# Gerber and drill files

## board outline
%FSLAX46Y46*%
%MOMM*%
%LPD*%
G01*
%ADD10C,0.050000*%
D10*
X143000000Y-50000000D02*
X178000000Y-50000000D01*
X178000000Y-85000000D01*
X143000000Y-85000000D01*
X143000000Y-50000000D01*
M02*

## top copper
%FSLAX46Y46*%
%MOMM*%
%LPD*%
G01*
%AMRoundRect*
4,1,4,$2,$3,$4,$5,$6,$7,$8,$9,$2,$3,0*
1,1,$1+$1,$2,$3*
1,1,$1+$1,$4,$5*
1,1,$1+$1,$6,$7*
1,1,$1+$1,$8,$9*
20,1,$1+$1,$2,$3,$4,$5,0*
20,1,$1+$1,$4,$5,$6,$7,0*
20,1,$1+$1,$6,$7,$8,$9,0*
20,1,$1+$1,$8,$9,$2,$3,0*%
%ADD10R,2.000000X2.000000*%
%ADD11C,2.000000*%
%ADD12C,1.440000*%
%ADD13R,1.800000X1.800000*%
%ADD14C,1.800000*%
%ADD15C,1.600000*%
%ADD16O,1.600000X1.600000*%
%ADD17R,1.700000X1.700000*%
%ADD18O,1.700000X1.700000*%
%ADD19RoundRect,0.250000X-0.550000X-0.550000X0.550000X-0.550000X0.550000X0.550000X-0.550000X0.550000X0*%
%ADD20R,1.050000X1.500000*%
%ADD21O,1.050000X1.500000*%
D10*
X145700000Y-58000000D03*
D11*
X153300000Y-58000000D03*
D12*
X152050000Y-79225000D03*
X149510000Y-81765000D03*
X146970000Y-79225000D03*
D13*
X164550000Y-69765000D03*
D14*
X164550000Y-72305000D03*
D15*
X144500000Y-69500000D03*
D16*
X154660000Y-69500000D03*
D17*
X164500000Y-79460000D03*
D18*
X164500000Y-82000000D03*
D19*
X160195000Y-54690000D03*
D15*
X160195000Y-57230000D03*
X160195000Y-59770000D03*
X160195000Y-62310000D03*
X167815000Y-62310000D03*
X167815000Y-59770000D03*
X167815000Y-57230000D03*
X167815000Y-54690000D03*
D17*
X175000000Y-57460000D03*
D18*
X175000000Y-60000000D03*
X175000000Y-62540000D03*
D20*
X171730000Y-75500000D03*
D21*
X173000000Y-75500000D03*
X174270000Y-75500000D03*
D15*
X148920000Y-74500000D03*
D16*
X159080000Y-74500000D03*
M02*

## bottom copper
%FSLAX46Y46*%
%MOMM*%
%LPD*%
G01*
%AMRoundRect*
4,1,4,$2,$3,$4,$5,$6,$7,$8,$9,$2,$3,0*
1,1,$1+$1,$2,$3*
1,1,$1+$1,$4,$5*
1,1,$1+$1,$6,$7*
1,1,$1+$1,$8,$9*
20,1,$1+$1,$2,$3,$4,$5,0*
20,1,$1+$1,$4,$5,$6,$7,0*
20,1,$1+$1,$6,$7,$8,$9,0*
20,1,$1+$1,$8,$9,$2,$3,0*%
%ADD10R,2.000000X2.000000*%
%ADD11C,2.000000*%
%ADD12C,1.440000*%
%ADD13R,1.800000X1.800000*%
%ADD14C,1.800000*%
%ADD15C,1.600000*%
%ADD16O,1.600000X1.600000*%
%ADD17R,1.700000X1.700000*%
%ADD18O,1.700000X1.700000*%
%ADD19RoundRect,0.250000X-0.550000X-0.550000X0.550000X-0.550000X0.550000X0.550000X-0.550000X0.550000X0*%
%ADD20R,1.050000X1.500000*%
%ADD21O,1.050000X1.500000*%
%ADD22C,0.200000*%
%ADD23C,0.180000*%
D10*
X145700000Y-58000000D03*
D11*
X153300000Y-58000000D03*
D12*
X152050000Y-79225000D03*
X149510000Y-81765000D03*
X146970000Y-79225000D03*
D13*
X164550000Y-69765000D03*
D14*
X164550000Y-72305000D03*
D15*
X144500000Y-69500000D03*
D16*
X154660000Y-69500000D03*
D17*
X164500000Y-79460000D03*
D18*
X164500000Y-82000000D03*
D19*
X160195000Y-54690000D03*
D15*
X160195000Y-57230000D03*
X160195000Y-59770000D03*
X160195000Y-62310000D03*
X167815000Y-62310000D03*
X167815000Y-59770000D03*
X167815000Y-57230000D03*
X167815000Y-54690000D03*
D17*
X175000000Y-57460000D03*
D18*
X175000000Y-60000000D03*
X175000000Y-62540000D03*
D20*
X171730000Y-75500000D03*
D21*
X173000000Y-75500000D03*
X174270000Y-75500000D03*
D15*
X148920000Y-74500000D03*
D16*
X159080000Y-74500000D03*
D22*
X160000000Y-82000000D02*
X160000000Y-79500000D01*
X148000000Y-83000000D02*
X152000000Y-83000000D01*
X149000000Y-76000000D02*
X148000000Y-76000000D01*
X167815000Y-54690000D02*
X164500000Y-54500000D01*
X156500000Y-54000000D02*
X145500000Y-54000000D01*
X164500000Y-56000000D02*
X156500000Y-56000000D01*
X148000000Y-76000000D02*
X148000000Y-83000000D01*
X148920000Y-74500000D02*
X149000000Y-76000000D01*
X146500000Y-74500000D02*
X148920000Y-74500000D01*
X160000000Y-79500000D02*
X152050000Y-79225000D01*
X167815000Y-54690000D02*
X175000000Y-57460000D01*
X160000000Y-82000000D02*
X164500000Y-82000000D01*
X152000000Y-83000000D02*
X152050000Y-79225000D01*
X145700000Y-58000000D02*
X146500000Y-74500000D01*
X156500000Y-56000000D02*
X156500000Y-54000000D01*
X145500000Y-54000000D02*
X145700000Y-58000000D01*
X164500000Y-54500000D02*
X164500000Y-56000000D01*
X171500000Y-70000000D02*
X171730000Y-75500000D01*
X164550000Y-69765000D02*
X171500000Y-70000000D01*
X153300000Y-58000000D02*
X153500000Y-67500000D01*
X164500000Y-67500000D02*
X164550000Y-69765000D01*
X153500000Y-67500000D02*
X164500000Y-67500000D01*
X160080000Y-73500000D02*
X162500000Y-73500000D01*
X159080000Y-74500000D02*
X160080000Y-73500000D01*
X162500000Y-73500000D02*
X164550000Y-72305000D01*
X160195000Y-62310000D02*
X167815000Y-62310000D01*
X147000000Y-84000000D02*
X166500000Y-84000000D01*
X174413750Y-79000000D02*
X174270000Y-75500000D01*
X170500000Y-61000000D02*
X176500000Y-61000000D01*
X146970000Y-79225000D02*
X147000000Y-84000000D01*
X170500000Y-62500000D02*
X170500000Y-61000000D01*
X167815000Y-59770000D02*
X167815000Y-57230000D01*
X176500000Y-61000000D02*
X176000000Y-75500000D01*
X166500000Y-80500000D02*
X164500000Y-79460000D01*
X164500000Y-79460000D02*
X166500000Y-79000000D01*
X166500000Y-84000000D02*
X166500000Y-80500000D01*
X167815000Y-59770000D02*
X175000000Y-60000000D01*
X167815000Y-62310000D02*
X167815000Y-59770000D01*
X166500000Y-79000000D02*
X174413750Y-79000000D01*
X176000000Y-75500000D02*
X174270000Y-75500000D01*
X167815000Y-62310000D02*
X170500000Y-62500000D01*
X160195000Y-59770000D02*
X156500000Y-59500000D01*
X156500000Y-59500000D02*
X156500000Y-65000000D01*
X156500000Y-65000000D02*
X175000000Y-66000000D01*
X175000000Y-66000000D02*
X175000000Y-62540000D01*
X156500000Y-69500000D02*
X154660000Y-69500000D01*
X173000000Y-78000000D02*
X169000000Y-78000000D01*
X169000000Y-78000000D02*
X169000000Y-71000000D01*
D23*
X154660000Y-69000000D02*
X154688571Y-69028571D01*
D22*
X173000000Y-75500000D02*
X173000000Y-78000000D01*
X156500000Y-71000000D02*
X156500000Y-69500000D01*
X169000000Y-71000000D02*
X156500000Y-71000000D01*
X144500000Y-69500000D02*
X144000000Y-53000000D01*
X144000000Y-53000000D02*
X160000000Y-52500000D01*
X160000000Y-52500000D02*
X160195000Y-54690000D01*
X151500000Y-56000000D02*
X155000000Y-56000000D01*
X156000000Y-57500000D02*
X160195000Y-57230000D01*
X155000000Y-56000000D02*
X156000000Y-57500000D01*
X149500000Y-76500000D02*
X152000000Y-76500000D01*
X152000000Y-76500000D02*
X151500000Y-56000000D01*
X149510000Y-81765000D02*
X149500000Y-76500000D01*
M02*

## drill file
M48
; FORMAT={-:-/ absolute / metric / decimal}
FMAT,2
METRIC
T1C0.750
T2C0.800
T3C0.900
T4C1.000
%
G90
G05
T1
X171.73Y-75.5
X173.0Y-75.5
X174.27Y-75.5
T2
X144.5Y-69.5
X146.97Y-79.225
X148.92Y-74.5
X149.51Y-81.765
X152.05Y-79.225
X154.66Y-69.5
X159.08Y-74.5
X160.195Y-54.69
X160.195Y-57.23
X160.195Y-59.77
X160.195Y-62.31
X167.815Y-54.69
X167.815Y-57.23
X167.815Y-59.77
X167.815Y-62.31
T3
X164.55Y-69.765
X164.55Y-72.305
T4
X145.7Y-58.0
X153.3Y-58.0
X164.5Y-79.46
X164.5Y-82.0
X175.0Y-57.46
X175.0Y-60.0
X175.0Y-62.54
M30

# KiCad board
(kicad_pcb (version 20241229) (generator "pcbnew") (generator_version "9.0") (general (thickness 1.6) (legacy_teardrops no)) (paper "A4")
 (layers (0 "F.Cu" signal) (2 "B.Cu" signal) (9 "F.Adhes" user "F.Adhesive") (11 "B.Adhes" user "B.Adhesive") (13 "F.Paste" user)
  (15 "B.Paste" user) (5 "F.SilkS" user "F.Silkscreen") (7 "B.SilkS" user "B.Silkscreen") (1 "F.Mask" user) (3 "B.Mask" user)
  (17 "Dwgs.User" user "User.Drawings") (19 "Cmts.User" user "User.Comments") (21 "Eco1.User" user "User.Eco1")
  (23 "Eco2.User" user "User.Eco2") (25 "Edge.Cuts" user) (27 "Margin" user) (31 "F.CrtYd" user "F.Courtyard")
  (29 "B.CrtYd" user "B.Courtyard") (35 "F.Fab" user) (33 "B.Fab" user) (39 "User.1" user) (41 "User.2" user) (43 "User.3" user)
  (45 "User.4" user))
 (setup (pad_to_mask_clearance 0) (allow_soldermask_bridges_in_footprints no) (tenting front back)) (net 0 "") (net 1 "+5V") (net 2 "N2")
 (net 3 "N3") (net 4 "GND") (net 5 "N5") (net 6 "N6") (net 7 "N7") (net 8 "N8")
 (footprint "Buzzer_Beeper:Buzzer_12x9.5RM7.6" (layer "F.Cu") (at 145.7 58)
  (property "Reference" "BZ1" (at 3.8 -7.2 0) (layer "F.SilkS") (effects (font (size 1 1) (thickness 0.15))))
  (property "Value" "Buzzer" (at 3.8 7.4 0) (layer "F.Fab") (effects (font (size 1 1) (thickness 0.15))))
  (pad "1" thru_hole rect (at 0 0) (size 2 2) (drill 1) (layers "*.Cu" "*.Mask") (remove_unused_layers no) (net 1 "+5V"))
  (pad "2" thru_hole circle (at 7.6 0) (size 2 2) (drill 1) (layers "*.Cu" "*.Mask") (remove_unused_layers no) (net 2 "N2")))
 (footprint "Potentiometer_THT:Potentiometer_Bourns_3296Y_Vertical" (layer "F.Cu") (at 152.05 79.225)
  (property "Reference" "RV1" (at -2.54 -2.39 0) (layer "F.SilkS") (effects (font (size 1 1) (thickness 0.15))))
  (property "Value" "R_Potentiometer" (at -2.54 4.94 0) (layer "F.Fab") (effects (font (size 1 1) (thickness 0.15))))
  (pad "1" thru_hole circle (at 0 0) (size 1.44 1.44) (drill 0.8) (layers "*.Cu" "*.Mask") (remove_unused_layers no) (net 1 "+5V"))
  (pad "2" thru_hole circle (at -2.54 2.54) (size 1.44 1.44) (drill 0.8) (layers "*.Cu" "*.Mask") (remove_unused_layers no) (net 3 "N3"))
  (pad "3" thru_hole circle (at -5.08 0) (size 1.44 1.44) (drill 0.8) (layers "*.Cu" "*.Mask") (remove_unused_layers no) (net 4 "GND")))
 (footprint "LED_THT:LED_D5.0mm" (layer "F.Cu") (at 164.55 69.765 -90)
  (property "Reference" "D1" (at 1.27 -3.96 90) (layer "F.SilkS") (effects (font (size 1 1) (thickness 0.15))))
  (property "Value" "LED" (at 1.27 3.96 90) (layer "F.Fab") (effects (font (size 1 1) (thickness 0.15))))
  (pad "1" thru_hole rect (at 0 0 270) (size 1.8 1.8) (drill 0.9) (layers "*.Cu" "*.Mask") (remove_unused_layers no) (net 2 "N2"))
  (pad "2" thru_hole circle (at 2.54 0 270) (size 1.8 1.8) (drill 0.9) (layers "*.Cu" "*.Mask") (remove_unused_layers no) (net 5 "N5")))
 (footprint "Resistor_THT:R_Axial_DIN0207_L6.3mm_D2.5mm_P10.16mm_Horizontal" (layer "F.Cu") (at 144.5 69.5)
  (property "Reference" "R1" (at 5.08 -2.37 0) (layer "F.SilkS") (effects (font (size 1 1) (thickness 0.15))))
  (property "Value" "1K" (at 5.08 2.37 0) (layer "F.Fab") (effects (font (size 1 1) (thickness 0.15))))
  (pad "1" thru_hole circle (at 0 0) (size 1.6 1.6) (drill 0.8) (layers "*.Cu" "*.Mask") (remove_unused_layers no) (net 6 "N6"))
  (pad "2" thru_hole oval (at 10.16 0) (size 1.6 1.6) (drill 0.8) (layers "*.Cu" "*.Mask") (remove_unused_layers no) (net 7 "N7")))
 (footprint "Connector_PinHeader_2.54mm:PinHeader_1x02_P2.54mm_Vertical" (layer "F.Cu") (at 164.5 79.46)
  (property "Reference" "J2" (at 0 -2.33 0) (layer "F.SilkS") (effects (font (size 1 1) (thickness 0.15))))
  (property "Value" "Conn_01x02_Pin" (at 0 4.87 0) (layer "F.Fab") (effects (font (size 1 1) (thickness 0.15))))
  (pad "1" thru_hole rect (at 0 0) (size 1.7 1.7) (drill 1) (layers "*.Cu" "*.Mask") (remove_unused_layers no) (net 4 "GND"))
  (pad "2" thru_hole oval (at 0 2.54) (size 1.7 1.7) (drill 1) (layers "*.Cu" "*.Mask") (remove_unused_layers no) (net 1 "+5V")))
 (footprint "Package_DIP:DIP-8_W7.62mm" (layer "F.Cu") (at 160.195 54.69)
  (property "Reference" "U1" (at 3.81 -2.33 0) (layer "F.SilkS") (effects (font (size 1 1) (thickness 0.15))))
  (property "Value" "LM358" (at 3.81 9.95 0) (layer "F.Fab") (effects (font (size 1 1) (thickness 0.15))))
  (pad "1" thru_hole roundrect (at 0 0) (size 1.6 1.6) (drill 0.8) (layers "*.Cu" "*.Mask") (remove_unused_layers no)
   (roundrect_rratio 0.15625) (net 6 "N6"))
  (pad "2" thru_hole circle (at 0 2.54) (size 1.6 1.6) (drill 0.8) (layers "*.Cu" "*.Mask") (remove_unused_layers no) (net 3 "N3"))
  (pad "3" thru_hole circle (at 0 5.08) (size 1.6 1.6) (drill 0.8) (layers "*.Cu" "*.Mask") (remove_unused_layers no) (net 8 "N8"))
  (pad "4" thru_hole circle (at 0 7.62) (size 1.6 1.6) (drill 0.8) (layers "*.Cu" "*.Mask") (remove_unused_layers no) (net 4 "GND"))
  (pad "5" thru_hole circle (at 7.62 7.62) (size 1.6 1.6) (drill 0.8) (layers "*.Cu" "*.Mask") (remove_unused_layers no) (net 4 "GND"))
  (pad "6" thru_hole circle (at 7.62 5.08) (size 1.6 1.6) (drill 0.8) (layers "*.Cu" "*.Mask") (remove_unused_layers no) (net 4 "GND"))
  (pad "7" thru_hole circle (at 7.62 2.54) (size 1.6 1.6) (drill 0.8) (layers "*.Cu" "*.Mask") (remove_unused_layers no) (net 4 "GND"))
  (pad "8" thru_hole circle (at 7.62 0) (size 1.6 1.6) (drill 0.8) (layers "*.Cu" "*.Mask") (remove_unused_layers no) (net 1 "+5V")))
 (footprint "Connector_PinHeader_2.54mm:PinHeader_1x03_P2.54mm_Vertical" (layer "F.Cu") (at 175 57.46)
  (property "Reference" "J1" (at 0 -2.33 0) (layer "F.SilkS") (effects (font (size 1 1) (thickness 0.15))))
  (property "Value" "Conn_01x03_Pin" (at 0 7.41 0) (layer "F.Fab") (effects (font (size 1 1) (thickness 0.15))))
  (pad "1" thru_hole rect (at 0 0) (size 1.7 1.7) (drill 1) (layers "*.Cu" "*.Mask") (remove_unused_layers no) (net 1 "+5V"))
  (pad "2" thru_hole oval (at 0 2.54) (size 1.7 1.7) (drill 1) (layers "*.Cu" "*.Mask") (remove_unused_layers no) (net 4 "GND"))
  (pad "3" thru_hole oval (at 0 5.08) (size 1.7 1.7) (drill 1) (layers "*.Cu" "*.Mask") (remove_unused_layers no) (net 8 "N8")))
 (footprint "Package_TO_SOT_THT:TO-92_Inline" (layer "F.Cu") (at 171.73 75.5)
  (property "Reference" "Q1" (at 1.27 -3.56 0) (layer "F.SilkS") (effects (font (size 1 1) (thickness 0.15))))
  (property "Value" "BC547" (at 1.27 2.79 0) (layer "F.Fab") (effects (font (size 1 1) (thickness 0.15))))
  (pad "1" thru_hole rect (at 0 0) (size 1.05 1.5) (drill 0.75) (layers "*.Cu" "*.Mask") (remove_unused_layers no) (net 2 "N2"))
  (pad "2" thru_hole oval (at 1.27 0) (size 1.05 1.5) (drill 0.75) (layers "*.Cu" "*.Mask") (remove_unused_layers no) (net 7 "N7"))
  (pad "3" thru_hole oval (at 2.54 0) (size 1.05 1.5) (drill 0.75) (layers "*.Cu" "*.Mask") (remove_unused_layers no) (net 4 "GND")))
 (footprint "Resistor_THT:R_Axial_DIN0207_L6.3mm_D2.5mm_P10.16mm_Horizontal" (layer "F.Cu") (at 148.92 74.5)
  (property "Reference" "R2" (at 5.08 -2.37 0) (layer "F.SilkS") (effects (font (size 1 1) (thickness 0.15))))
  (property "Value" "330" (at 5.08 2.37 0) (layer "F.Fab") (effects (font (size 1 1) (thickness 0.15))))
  (pad "1" thru_hole circle (at 0 0) (size 1.6 1.6) (drill 0.8) (layers "*.Cu" "*.Mask") (remove_unused_layers no) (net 1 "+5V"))
  (pad "2" thru_hole oval (at 10.16 0) (size 1.6 1.6) (drill 0.8) (layers "*.Cu" "*.Mask") (remove_unused_layers no) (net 5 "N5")))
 (gr_rect (start 178 85) (end 143 50) (stroke (width 0.05) (type solid)) (fill no) (layer "Edge.Cuts"))
 (segment (start 160 82) (end 160 79.5) (width 0.2) (layer "B.Cu") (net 1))
 (segment (start 148 83) (end 152 83) (width 0.2) (layer "B.Cu") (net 1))
 (segment (start 149 76) (end 148 76) (width 0.2) (layer "B.Cu") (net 1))
 (segment (start 167.815 54.69) (end 164.5 54.5) (width 0.2) (layer "B.Cu") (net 1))
 (segment (start 156.5 54) (end 145.5 54) (width 0.2) (layer "B.Cu") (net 1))
 (segment (start 164.5 56) (end 156.5 56) (width 0.2) (layer "B.Cu") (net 1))
 (segment (start 148 76) (end 148 83) (width 0.2) (layer "B.Cu") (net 1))
 (segment (start 148.92 74.5) (end 149 76) (width 0.2) (layer "B.Cu") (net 1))
 (segment (start 146.5 74.5) (end 148.92 74.5) (width 0.2) (layer "B.Cu") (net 1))
 (segment (start 160 79.5) (end 152.05 79.225) (width 0.2) (layer "B.Cu") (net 1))
 (segment (start 167.815 54.69) (end 175 57.46) (width 0.2) (layer "B.Cu") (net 1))
 (segment (start 160 82) (end 164.5 82) (width 0.2) (layer "B.Cu") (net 1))
 (segment (start 152 83) (end 152.05 79.225) (width 0.2) (layer "B.Cu") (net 1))
 (segment (start 145.7 58) (end 146.5 74.5) (width 0.2) (layer "B.Cu") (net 1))
 (segment (start 156.5 56) (end 156.5 54) (width 0.2) (layer "B.Cu") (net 1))
 (segment (start 145.5 54) (end 145.7 58) (width 0.2) (layer "B.Cu") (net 1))
 (segment (start 164.5 54.5) (end 164.5 56) (width 0.2) (layer "B.Cu") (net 1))
 (segment (start 171.5 70) (end 171.73 75.5) (width 0.2) (layer "B.Cu") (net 2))
 (segment (start 164.55 69.765) (end 171.5 70) (width 0.2) (layer "B.Cu") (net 2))
 (segment (start 153.3 58) (end 153.5 67.5) (width 0.2) (layer "B.Cu") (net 2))
 (segment (start 164.5 67.5) (end 164.55 69.765) (width 0.2) (layer "B.Cu") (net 2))
 (segment (start 153.5 67.5) (end 164.5 67.5) (width 0.2) (layer "B.Cu") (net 2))
 (segment (start 160.08 73.5) (end 162.5 73.5) (width 0.2) (layer "B.Cu") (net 5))
 (segment (start 159.08 74.5) (end 160.08 73.5) (width 0.2) (layer "B.Cu") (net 5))
 (segment (start 162.5 73.5) (end 164.55 72.305) (width 0.2) (layer "B.Cu") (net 5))
 (segment (start 160.195 62.31) (end 167.815 62.31) (width 0.2) (layer "B.Cu") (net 4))
 (segment (start 147 84) (end 166.5 84) (width 0.2) (layer "B.Cu") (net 4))
 (segment (start 174.41375 79) (end 174.27 75.5) (width 0.2) (layer "B.Cu") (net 4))
 (segment (start 170.5 61) (end 176.5 61) (width 0.2) (layer "B.Cu") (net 4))
 (segment (start 146.97 79.225) (end 147 84) (width 0.2) (layer "B.Cu") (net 4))
 (segment (start 170.5 62.5) (end 170.5 61) (width 0.2) (layer "B.Cu") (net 4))
 (segment (start 167.815 59.77) (end 167.815 57.23) (width 0.2) (layer "B.Cu") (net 4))
 (segment (start 176.5 61) (end 176 75.5) (width 0.2) (layer "B.Cu") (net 4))
 (segment (start 166.5 80.5) (end 164.5 79.46) (width 0.2) (layer "B.Cu") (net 4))
 (segment (start 164.5 79.46) (end 166.5 79) (width 0.2) (layer "B.Cu") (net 4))
 (segment (start 166.5 84) (end 166.5 80.5) (width 0.2) (layer "B.Cu") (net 4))
 (segment (start 167.815 59.77) (end 175 60) (width 0.2) (layer "B.Cu") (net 4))
 (segment (start 167.815 62.31) (end 167.815 59.77) (width 0.2) (layer "B.Cu") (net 4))
 (segment (start 166.5 79) (end 174.41375 79) (width 0.2) (layer "B.Cu") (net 4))
 (segment (start 176 75.5) (end 174.27 75.5) (width 0.2) (layer "B.Cu") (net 4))
 (segment (start 167.815 62.31) (end 170.5 62.5) (width 0.2) (layer "B.Cu") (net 4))
 (segment (start 160.195 59.77) (end 156.5 59.5) (width 0.2) (layer "B.Cu") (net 8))
 (segment (start 156.5 59.5) (end 156.5 65) (width 0.2) (layer "B.Cu") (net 8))
 (segment (start 156.5 65) (end 175 66) (width 0.2) (layer "B.Cu") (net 8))
 (segment (start 175 66) (end 175 62.54) (width 0.2) (layer "B.Cu") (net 8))
 (segment (start 156.5 69.5) (end 154.66 69.5) (width 0.2) (layer "B.Cu") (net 7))
 (segment (start 173 78) (end 169 78) (width 0.2) (layer "B.Cu") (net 7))
 (segment (start 169 78) (end 169 71) (width 0.2) (layer "B.Cu") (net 7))
 (segment (start 154.66 69) (end 154.688571 69.028571) (width 0.18) (layer "B.Cu") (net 7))
 (segment (start 173 75.5) (end 173 78) (width 0.2) (layer "B.Cu") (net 7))
 (segment (start 156.5 71) (end 156.5 69.5) (width 0.2) (layer "B.Cu") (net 7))
 (segment (start 169 71) (end 156.5 71) (width 0.2) (layer "B.Cu") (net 7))
 (segment (start 144.5 69.5) (end 144 53) (width 0.2) (layer "B.Cu") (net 6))
 (segment (start 144 53) (end 160 52.5) (width 0.2) (layer "B.Cu") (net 6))
 (segment (start 160 52.5) (end 160.195 54.69) (width 0.2) (layer "B.Cu") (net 6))
 (segment (start 151.5 56) (end 155 56) (width 0.2) (layer "B.Cu") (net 3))
 (segment (start 156 57.5) (end 160.195 57.23) (width 0.2) (layer "B.Cu") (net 3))
 (segment (start 155 56) (end 156 57.5) (width 0.2) (layer "B.Cu") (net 3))
 (segment (start 149.5 76.5) (end 152 76.5) (width 0.2) (layer "B.Cu") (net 3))
 (segment (start 152 76.5) (end 151.5 56) (width 0.2) (layer "B.Cu") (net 3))
 (segment (start 149.51 81.765) (end 149.5 76.5) (width 0.2) (layer "B.Cu") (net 3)))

